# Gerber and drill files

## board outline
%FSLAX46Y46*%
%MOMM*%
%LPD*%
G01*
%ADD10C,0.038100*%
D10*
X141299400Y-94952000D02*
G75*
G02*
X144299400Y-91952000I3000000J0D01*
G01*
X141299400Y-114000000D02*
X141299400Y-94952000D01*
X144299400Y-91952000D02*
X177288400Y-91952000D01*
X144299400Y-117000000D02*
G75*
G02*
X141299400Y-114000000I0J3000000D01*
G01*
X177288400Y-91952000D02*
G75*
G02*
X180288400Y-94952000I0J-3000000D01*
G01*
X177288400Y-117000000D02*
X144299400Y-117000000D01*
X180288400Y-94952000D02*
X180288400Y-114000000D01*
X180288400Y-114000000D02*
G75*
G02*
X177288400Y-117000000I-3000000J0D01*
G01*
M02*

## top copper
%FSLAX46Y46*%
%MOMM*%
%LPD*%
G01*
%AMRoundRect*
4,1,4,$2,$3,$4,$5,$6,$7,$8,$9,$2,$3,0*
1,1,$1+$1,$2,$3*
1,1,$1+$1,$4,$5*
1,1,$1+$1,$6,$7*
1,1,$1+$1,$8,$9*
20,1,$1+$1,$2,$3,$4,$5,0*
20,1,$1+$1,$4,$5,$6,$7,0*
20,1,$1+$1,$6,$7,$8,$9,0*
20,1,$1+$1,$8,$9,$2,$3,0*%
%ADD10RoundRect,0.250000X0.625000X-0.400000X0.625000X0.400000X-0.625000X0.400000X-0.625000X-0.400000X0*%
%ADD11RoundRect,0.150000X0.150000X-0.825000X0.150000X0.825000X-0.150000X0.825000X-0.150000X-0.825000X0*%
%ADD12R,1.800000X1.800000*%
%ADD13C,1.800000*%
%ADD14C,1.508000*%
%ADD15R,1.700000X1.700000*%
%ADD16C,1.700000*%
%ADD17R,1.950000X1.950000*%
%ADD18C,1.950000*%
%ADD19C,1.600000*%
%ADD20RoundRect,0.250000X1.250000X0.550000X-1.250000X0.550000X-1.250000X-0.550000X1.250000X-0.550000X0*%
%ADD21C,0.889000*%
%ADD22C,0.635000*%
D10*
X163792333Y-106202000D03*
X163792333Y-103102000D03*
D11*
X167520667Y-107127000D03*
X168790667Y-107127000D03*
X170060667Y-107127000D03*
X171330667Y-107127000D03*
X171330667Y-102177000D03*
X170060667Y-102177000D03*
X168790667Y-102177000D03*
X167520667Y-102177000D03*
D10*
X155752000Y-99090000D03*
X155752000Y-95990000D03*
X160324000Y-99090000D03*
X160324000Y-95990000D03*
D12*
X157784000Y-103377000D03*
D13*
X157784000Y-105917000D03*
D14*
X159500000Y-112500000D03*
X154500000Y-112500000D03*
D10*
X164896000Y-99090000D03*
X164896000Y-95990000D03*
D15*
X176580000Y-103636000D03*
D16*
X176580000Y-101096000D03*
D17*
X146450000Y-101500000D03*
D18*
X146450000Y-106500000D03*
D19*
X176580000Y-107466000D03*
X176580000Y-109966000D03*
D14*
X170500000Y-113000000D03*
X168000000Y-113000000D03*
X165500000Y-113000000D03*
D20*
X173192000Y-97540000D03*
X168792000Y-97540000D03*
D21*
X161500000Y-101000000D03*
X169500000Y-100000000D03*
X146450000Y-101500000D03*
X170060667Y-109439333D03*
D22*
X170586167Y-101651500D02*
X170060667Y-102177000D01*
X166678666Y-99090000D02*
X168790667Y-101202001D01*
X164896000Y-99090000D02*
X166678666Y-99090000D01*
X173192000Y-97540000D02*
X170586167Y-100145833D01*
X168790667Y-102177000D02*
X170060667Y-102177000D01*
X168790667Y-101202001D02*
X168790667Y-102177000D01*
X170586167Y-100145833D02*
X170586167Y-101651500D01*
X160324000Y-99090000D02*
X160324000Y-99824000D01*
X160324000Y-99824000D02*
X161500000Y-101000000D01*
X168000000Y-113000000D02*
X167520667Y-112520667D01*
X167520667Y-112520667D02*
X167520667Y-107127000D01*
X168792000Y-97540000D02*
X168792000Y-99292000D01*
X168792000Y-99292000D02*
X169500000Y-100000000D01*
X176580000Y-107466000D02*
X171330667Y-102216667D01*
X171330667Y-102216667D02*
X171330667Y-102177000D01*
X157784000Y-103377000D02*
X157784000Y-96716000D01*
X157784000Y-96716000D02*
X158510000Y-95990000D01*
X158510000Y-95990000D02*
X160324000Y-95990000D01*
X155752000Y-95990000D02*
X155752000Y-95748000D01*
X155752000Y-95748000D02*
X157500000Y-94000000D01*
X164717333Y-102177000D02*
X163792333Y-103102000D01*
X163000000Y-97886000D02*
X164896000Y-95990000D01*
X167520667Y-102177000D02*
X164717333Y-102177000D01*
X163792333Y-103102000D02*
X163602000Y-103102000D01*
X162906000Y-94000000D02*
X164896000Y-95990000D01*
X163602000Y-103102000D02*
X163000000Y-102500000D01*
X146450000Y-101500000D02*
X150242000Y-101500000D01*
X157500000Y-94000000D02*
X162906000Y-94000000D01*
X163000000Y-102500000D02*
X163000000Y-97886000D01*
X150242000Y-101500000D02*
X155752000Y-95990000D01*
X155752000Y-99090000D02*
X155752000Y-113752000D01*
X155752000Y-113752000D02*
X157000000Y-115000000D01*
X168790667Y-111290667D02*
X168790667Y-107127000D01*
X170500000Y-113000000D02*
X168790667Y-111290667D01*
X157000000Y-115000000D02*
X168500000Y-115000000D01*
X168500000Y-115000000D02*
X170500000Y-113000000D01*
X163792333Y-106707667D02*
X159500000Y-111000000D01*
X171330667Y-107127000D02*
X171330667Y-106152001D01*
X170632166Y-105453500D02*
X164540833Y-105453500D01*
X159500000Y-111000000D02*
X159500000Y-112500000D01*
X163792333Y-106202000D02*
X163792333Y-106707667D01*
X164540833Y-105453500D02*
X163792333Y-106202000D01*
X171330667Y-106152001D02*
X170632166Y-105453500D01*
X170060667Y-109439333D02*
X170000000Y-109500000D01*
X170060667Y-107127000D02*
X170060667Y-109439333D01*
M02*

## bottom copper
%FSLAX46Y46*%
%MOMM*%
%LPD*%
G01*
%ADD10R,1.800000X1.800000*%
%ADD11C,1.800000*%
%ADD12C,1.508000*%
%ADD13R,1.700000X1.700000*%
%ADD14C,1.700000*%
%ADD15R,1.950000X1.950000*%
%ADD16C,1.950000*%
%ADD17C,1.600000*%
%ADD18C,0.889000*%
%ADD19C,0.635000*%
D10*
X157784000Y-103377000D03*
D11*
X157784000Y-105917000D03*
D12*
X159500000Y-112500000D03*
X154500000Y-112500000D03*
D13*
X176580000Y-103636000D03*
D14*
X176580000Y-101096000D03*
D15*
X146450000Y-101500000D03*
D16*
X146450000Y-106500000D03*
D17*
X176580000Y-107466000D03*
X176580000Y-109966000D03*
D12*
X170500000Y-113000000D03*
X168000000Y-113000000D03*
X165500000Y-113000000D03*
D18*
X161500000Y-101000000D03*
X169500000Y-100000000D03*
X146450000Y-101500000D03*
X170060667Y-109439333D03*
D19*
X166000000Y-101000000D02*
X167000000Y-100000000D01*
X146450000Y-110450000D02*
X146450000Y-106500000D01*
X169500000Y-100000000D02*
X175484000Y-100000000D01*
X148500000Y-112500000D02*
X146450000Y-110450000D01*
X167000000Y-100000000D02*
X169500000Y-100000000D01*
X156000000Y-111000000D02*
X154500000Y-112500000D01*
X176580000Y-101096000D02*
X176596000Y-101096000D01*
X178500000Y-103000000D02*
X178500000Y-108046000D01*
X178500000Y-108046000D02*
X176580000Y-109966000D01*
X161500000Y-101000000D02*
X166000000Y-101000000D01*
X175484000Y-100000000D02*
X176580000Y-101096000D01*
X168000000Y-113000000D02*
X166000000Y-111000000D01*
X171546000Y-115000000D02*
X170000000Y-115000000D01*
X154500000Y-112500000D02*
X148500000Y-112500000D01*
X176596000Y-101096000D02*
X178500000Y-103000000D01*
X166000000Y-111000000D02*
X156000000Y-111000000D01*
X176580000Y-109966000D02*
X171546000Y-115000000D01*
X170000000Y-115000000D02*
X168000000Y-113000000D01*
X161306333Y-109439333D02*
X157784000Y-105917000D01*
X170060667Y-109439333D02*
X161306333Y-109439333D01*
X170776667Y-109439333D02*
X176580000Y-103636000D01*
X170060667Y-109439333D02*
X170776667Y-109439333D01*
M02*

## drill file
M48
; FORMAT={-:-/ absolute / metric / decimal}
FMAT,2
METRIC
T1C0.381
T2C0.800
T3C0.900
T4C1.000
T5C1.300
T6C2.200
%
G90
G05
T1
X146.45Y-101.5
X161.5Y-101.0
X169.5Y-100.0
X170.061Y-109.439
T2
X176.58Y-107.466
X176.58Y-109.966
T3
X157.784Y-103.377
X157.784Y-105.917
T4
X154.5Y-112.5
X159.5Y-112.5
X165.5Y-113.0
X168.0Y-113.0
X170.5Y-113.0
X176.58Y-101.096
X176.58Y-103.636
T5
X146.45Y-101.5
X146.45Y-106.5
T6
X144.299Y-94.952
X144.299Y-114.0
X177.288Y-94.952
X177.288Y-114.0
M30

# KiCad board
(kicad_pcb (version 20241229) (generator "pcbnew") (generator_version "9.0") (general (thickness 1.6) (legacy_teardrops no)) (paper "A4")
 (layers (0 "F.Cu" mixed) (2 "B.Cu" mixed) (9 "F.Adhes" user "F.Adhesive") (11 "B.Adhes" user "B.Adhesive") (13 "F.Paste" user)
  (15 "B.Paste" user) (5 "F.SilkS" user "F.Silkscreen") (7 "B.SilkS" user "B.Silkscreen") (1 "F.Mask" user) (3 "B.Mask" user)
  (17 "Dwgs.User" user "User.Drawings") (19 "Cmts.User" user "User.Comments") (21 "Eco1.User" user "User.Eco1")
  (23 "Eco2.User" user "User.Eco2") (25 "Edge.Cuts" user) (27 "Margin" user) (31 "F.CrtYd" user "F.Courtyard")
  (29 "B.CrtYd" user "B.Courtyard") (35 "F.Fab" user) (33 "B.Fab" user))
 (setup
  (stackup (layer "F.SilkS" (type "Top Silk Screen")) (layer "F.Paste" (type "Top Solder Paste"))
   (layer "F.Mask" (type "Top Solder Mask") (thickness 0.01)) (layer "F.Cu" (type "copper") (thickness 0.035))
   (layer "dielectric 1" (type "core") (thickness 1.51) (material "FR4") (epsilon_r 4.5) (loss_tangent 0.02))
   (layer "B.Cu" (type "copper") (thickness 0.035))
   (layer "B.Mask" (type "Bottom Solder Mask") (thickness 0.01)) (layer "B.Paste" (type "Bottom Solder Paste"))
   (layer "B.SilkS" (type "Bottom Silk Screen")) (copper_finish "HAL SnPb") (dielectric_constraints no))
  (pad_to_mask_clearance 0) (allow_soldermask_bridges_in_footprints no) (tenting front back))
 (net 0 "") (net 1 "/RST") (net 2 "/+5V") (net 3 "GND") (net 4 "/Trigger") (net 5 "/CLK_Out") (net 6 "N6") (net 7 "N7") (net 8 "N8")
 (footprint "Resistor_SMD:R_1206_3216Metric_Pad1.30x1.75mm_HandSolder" (layer "F.Cu") (at 163.792333 104.652 90)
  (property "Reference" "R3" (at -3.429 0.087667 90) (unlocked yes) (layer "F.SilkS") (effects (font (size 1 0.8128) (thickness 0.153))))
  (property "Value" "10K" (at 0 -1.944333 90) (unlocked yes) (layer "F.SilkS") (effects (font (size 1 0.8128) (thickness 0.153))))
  (pad "1" smd roundrect (at -1.55 0 90) (size 1.3 1.75) (layers "F.Cu" "F.Mask" "F.Paste") (roundrect_rratio 0.192308) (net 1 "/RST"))
  (pad "2" smd roundrect (at 1.55 0 90) (size 1.3 1.75) (layers "F.Cu" "F.Mask" "F.Paste") (roundrect_rratio 0.192308) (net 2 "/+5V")))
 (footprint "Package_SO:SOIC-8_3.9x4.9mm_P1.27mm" (layer "F.Cu") (at 169.425667 104.652 90)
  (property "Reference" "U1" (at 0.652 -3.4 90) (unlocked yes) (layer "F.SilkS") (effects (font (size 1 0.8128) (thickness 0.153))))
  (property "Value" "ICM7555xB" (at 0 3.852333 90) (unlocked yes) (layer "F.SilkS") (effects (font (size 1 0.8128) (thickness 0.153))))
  (pad "1" smd roundrect (at -2.475 -1.905 90) (size 1.95 0.6) (layers "F.Cu" "F.Mask" "F.Paste") (roundrect_rratio 0.25) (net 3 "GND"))
  (pad "2" smd roundrect (at -2.475 -0.635 90) (size 1.95 0.6) (layers "F.Cu" "F.Mask" "F.Paste") (roundrect_rratio 0.25) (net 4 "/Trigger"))
  (pad "3" smd roundrect (at -2.475 0.635 90) (size 1.95 0.6) (layers "F.Cu" "F.Mask" "F.Paste") (roundrect_rratio 0.25) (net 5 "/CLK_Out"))
  (pad "4" smd roundrect (at -2.475 1.905 90) (size 1.95 0.6) (layers "F.Cu" "F.Mask" "F.Paste") (roundrect_rratio 0.25) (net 1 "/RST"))
  (pad "5" smd roundrect (at 2.475 1.905 90) (size 1.95 0.6) (layers "F.Cu" "F.Mask" "F.Paste") (roundrect_rratio 0.25) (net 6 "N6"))
  (pad "6" smd roundrect (at 2.475 0.635 90) (size 1.95 0.6) (layers "F.Cu" "F.Mask" "F.Paste") (roundrect_rratio 0.25) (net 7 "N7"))
  (pad "7" smd roundrect (at 2.475 -0.635 90) (size 1.95 0.6) (layers "F.Cu" "F.Mask" "F.Paste") (roundrect_rratio 0.25) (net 7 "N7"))
  (pad "8" smd roundrect (at 2.475 -1.905 90) (size 1.95 0.6) (layers "F.Cu" "F.Mask" "F.Paste") (roundrect_rratio 0.25) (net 2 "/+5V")))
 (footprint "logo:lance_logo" (layer "F.Cu") (at 149.5 95.5)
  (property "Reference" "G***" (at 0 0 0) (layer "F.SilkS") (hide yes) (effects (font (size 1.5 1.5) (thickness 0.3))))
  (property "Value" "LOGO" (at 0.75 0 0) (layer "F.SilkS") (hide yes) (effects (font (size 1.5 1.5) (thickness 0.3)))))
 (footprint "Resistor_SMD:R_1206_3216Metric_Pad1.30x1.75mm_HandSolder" (layer "F.Cu") (at 155.752 97.54 90)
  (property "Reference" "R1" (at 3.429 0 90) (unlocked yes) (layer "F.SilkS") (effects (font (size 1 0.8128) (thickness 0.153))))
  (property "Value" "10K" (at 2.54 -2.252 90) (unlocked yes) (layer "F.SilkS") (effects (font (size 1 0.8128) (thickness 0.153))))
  (pad "1" smd roundrect (at -1.55 0 90) (size 1.3 1.75) (layers "F.Cu" "F.Mask" "F.Paste") (roundrect_rratio 0.192308) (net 4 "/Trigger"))
  (pad "2" smd roundrect (at 1.55 0 90) (size 1.3 1.75) (layers "F.Cu" "F.Mask" "F.Paste") (roundrect_rratio 0.192308) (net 2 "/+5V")))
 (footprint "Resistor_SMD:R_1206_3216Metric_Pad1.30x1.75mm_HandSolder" (layer "F.Cu") (at 160.324 97.54 90)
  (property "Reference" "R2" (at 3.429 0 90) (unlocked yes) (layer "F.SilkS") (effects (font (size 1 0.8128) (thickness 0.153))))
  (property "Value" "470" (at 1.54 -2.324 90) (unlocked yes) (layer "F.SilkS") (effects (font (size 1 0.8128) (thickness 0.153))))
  (pad "1" smd roundrect (at -1.55 0 90) (size 1.3 1.75) (layers "F.Cu" "F.Mask" "F.Paste") (roundrect_rratio 0.192308) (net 3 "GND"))
  (pad "2" smd roundrect (at 1.55 0 90) (size 1.3 1.75) (layers "F.Cu" "F.Mask" "F.Paste") (roundrect_rratio 0.192308) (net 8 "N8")))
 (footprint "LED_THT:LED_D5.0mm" (layer "F.Cu") (at 157.784 103.377 -90)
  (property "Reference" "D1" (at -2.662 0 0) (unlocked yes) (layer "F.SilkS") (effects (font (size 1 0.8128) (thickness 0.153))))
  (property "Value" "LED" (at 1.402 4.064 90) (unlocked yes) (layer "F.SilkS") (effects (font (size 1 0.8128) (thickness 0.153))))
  (pad "1" thru_hole rect (at 0 0 270) (size 1.8 1.8) (drill 0.9) (layers "*.Cu" "*.Mask") (remove_unused_layers no) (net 8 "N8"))
  (pad "2" thru_hole circle (at 2.54 0 270) (size 1.8 1.8) (drill 0.9) (layers "*.Cu" "*.Mask") (remove_unused_layers no) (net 5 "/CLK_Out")))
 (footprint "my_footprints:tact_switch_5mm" (layer "F.Cu") (at 157 112.5 180)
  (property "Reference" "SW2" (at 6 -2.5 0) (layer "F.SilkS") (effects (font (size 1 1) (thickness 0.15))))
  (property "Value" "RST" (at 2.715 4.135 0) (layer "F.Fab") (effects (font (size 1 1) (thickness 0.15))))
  (pad "1" thru_hole circle (at -2.5 0 180) (size 1.508 1.508) (drill 1) (layers "*.Cu" "*.Mask") (remove_unused_layers no) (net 1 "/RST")
   (solder_mask_margin 0.102))
  (pad "2" thru_hole circle (at 2.5 0 180) (size 1.508 1.508) (drill 1) (layers "*.Cu" "*.Mask") (remove_unused_layers no) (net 3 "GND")
   (solder_mask_margin 0.102)))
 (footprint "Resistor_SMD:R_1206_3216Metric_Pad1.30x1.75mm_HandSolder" (layer "F.Cu") (at 164.896 97.54 90)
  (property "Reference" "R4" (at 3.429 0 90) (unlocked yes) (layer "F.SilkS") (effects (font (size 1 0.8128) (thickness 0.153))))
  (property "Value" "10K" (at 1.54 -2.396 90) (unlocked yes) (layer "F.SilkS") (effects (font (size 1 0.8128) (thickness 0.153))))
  (pad "1" smd roundrect (at -1.55 0 90) (size 1.3 1.75) (layers "F.Cu" "F.Mask" "F.Paste") (roundrect_rratio 0.192308) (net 7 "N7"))
  (pad "2" smd roundrect (at 1.55 0 90) (size 1.3 1.75) (layers "F.Cu" "F.Mask" "F.Paste") (roundrect_rratio 0.192308) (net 2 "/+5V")))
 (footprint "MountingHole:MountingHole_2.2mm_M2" (layer "F.Cu") (at 144.2994 94.952)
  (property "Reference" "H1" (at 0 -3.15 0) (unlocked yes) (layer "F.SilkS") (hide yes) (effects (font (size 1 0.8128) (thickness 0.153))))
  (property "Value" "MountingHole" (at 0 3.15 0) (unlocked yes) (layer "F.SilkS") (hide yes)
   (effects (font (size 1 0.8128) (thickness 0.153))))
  (pad "" np_thru_hole circle (at 0 0) (size 2.2 2.2) (drill 2.2) (layers "*.Cu" "*.Mask")))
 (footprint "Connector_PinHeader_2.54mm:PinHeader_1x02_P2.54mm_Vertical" (layer "F.Cu") (at 176.58 103.636 180)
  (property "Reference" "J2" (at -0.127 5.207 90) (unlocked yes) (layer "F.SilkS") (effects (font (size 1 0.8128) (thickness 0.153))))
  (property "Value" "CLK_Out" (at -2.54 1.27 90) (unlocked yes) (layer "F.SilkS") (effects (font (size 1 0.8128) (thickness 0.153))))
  (pad "1" thru_hole rect (at 0 0 180) (size 1.7 1.7) (drill 1) (layers "*.Cu" "*.Mask") (remove_unused_layers no) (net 5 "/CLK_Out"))
  (pad "2" thru_hole circle (at 0 2.54 180) (size 1.7 1.7) (drill 1) (layers "*.Cu" "*.Mask") (remove_unused_layers no) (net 3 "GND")))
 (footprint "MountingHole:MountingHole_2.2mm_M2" (layer "F.Cu") (at 177.2884 114)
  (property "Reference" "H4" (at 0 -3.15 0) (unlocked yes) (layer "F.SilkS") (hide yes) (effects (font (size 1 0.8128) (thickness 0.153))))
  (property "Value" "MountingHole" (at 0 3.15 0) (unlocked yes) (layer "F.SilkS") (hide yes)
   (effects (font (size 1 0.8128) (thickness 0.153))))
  (pad "" np_thru_hole circle (at 0 0) (size 2.2 2.2) (drill 2.2) (layers "*.Cu" "*.Mask")))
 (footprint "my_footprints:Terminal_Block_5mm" (layer "F.Cu") (at 146.45 104 -90)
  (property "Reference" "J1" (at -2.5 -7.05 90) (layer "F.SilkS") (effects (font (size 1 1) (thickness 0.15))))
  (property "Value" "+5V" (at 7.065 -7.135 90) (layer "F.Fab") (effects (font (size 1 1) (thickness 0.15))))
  (pad "1" thru_hole rect (at -2.5 0 270) (size 1.95 1.95) (drill 1.3) (layers "*.Cu" "*.Mask") (remove_unused_layers no) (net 2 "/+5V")
   (solder_mask_margin 0.102))
  (pad "2" thru_hole circle (at 2.5 0 270) (size 1.95 1.95) (drill 1.3) (layers "*.Cu" "*.Mask") (remove_unused_layers no) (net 3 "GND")
   (solder_mask_margin 0.102)))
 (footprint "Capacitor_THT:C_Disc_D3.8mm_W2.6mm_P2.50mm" (layer "F.Cu") (at 176.58 107.466 -90)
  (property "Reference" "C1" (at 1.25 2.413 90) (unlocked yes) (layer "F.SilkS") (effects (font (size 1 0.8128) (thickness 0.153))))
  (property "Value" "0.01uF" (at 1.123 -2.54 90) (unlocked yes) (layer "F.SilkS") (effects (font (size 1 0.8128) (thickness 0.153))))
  (pad "1" thru_hole circle (at 0 0 270) (size 1.6 1.6) (drill 0.8) (layers "*.Cu" "*.Mask") (remove_unused_layers no) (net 6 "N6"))
  (pad "2" thru_hole circle (at 2.5 0 270) (size 1.6 1.6) (drill 0.8) (layers "*.Cu" "*.Mask") (remove_unused_layers no) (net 3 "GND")))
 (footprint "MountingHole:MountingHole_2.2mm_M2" (layer "F.Cu") (at 177.2884 94.952)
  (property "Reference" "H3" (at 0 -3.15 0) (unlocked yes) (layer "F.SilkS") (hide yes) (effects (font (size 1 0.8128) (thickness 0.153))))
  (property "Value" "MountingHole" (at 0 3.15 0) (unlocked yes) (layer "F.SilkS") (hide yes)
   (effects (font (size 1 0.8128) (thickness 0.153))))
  (pad "" np_thru_hole circle (at 0 0) (size 2.2 2.2) (drill 2.2) (layers "*.Cu" "*.Mask")))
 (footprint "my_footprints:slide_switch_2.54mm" (layer "F.Cu") (at 168 113 180)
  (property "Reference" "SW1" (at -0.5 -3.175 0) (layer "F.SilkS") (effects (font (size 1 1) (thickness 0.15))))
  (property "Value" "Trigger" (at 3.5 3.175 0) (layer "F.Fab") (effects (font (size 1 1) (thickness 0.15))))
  (pad "1" thru_hole circle (at -2.5 0 180) (size 1.508 1.508) (drill 1) (layers "*.Cu" "*.Mask") (remove_unused_layers no)
   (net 4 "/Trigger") (solder_mask_margin 0.102))
  (pad "2" thru_hole circle (at 0 0 180) (size 1.508 1.508) (drill 1) (layers "*.Cu" "*.Mask") (remove_unused_layers no) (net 3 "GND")
   (solder_mask_margin 0.102))
  (pad "3" thru_hole circle (at 2.5 0 180) (size 1.508 1.508) (drill 1) (layers "*.Cu" "*.Mask") (remove_unused_layers no)
   (solder_mask_margin 0.102)))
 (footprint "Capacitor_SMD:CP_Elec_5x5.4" (layer "F.Cu") (at 170.992 97.54 180)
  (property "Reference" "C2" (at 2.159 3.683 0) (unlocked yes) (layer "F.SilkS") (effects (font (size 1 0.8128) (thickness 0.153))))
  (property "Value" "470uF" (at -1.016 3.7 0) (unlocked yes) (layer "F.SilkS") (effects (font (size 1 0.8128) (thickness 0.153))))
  (pad "1" smd roundrect (at -2.2 0 180) (size 3 1.6) (layers "F.Cu" "F.Mask" "F.Paste") (roundrect_rratio 0.15625) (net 7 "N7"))
  (pad "2" smd roundrect (at 2.2 0 180) (size 3 1.6) (layers "F.Cu" "F.Mask" "F.Paste") (roundrect_rratio 0.15625) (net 3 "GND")))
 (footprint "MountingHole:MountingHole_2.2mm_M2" (layer "F.Cu") (at 144.2994 114)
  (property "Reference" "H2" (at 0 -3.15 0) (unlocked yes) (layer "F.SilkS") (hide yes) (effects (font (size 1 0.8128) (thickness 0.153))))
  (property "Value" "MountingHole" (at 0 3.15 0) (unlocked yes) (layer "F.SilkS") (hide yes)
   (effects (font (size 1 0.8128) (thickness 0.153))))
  (pad "" np_thru_hole circle (at 0 0) (size 2.2 2.2) (drill 2.2) (layers "*.Cu" "*.Mask")))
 (gr_arc (start 141.2994 94.952) (mid 142.17808 92.83068) (end 144.2994 91.952) (stroke (width 0.0381) (type default)) (layer "Edge.Cuts"))
 (gr_line (start 141.2994 114) (end 141.2994 94.952) (stroke (width 0.0381) (type default)) (layer "Edge.Cuts"))
 (gr_line (start 144.2994 91.952) (end 177.2884 91.952) (stroke (width 0.0381) (type default)) (layer "Edge.Cuts"))
 (gr_arc (start 144.2994 117) (mid 142.17808 116.12132) (end 141.2994 114) (stroke (width 0.0381) (type default)) (layer "Edge.Cuts"))
 (gr_arc (start 177.2884 91.952) (mid 179.40972 92.83068) (end 180.2884 94.952) (stroke (width 0.0381) (type default)) (layer "Edge.Cuts"))
 (gr_line (start 177.2884 117) (end 144.2994 117) (stroke (width 0.0381) (type default)) (layer "Edge.Cuts"))
 (gr_line (start 180.2884 94.952) (end 180.2884 114) (stroke (width 0.0381) (type default)) (layer "Edge.Cuts"))
 (gr_arc (start 180.2884 114) (mid 179.40972 116.12132) (end 177.2884 117) (stroke (width 0.0381) (type default)) (layer "Edge.Cuts"))
 (segment (start 170.586167 101.6515) (end 170.060667 102.177) (width 0.635) (layer "F.Cu") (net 7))
 (segment (start 166.678666 99.09) (end 168.790667 101.202001) (width 0.635) (layer "F.Cu") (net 7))
 (segment (start 164.896 99.09) (end 166.678666 99.09) (width 0.635) (layer "F.Cu") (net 7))
 (segment (start 173.192 97.54) (end 170.586167 100.145833) (width 0.635) (layer "F.Cu") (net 7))
 (segment (start 168.790667 102.177) (end 170.060667 102.177) (width 0.635) (layer "F.Cu") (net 7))
 (segment (start 168.790667 101.202001) (end 168.790667 102.177) (width 0.635) (layer "F.Cu") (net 7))
 (segment (start 170.586167 100.145833) (end 170.586167 101.6515) (width 0.635) (layer "F.Cu") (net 7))
 (segment (start 160.324 99.09) (end 160.324 99.824) (width 0.635) (layer "F.Cu") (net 3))
 (segment (start 160.324 99.824) (end 161.5 101) (width 0.635) (layer "F.Cu") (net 3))
 (segment (start 168 113) (end 167.520667 112.520667) (width 0.635) (layer "F.Cu") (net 3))
 (segment (start 167.520667 112.520667) (end 167.520667 107.127) (width 0.635) (layer "F.Cu") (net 3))
 (segment (start 168.792 97.54) (end 168.792 99.292) (width 0.635) (layer "F.Cu") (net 3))
 (segment (start 168.792 99.292) (end 169.5 100) (width 0.635) (layer "F.Cu") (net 3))
 (via (at 161.5 101) (size 0.889) (drill 0.381) (layers "F.Cu" "B.Cu") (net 3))
 (via (at 169.5 100) (size 0.889) (drill 0.381) (layers "F.Cu" "B.Cu") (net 3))
 (segment (start 166 101) (end 167 100) (width 0.635) (layer "B.Cu") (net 3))
 (segment (start 146.45 110.45) (end 146.45 106.5) (width 0.635) (layer "B.Cu") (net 3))
 (segment (start 169.5 100) (end 175.484 100) (width 0.635) (layer "B.Cu") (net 3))
 (segment (start 148.5 112.5) (end 146.45 110.45) (width 0.635) (layer "B.Cu") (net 3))
 (segment (start 167 100) (end 169.5 100) (width 0.635) (layer "B.Cu") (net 3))
 (segment (start 156 111) (end 154.5 112.5) (width 0.635) (layer "B.Cu") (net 3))
 (segment (start 176.58 101.096) (end 176.596 101.096) (width 0.635) (layer "B.Cu") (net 3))
 (segment (start 178.5 103) (end 178.5 108.046) (width 0.635) (layer "B.Cu") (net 3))
 (segment (start 178.5 108.046) (end 176.58 109.966) (width 0.635) (layer "B.Cu") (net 3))
 (segment (start 161.5 101) (end 166 101) (width 0.635) (layer "B.Cu") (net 3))
 (segment (start 175.484 100) (end 176.58 101.096) (width 0.635) (layer "B.Cu") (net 3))
 (segment (start 168 113) (end 166 111) (width 0.635) (layer "B.Cu") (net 3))
 (segment (start 171.546 115) (end 170 115) (width 0.635) (layer "B.Cu") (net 3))
 (segment (start 154.5 112.5) (end 148.5 112.5) (width 0.635) (layer "B.Cu") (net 3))
 (segment (start 176.596 101.096) (end 178.5 103) (width 0.635) (layer "B.Cu") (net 3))
 (segment (start 166 111) (end 156 111) (width 0.635) (layer "B.Cu") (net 3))
 (segment (start 176.58 109.966) (end 171.546 115) (width 0.635) (layer "B.Cu") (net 3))
 (segment (start 170 115) (end 168 113) (width 0.635) (layer "B.Cu") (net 3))
 (segment (start 176.58 107.466) (end 171.330667 102.216667) (width 0.635) (layer "F.Cu") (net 6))
 (segment (start 171.330667 102.216667) (end 171.330667 102.177) (width 0.635) (layer "F.Cu") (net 6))
 (segment (start 157.784 103.377) (end 157.784 96.716) (width 0.635) (layer "F.Cu") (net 8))
 (segment (start 157.784 96.716) (end 158.51 95.99) (width 0.635) (layer "F.Cu") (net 8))
 (segment (start 158.51 95.99) (end 160.324 95.99) (width 0.635) (layer "F.Cu") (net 8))
 (segment (start 155.752 95.99) (end 155.752 95.748) (width 0.635) (layer "F.Cu") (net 2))
 (segment (start 155.752 95.748) (end 157.5 94) (width 0.635) (layer "F.Cu") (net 2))
 (segment (start 164.717333 102.177) (end 163.792333 103.102) (width 0.635) (layer "F.Cu") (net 2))
 (segment (start 163 97.886) (end 164.896 95.99) (width 0.635) (layer "F.Cu") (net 2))
 (segment (start 167.520667 102.177) (end 164.717333 102.177) (width 0.635) (layer "F.Cu") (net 2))
 (segment (start 163.792333 103.102) (end 163.602 103.102) (width 0.635) (layer "F.Cu") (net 2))
 (segment (start 162.906 94) (end 164.896 95.99) (width 0.635) (layer "F.Cu") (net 2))
 (segment (start 163.602 103.102) (end 163 102.5) (width 0.635) (layer "F.Cu") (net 2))
 (segment (start 146.45 101.5) (end 150.242 101.5) (width 0.635) (layer "F.Cu") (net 2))
 (segment (start 157.5 94) (end 162.906 94) (width 0.635) (layer "F.Cu") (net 2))
 (segment (start 163 102.5) (end 163 97.886) (width 0.635) (layer "F.Cu") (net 2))
 (segment (start 150.242 101.5) (end 155.752 95.99) (width 0.635) (layer "F.Cu") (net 2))
 (via (at 146.45 101.5) (size 0.889) (drill 0.381) (layers "F.Cu" "B.Cu") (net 2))
 (segment (start 155.752 99.09) (end 155.752 113.752) (width 0.635) (layer "F.Cu") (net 4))
 (segment (start 155.752 113.752) (end 157 115) (width 0.635) (layer "F.Cu") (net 4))
 (segment (start 168.790667 111.290667) (end 168.790667 107.127) (width 0.635) (layer "F.Cu") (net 4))
 (segment (start 170.5 113) (end 168.790667 111.290667) (width 0.635) (layer "F.Cu") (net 4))
 (segment (start 157 115) (end 168.5 115) (width 0.635) (layer "F.Cu") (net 4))
 (segment (start 168.5 115) (end 170.5 113) (width 0.635) (layer "F.Cu") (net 4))
 (segment (start 163.792333 106.707667) (end 159.5 111) (width 0.635) (layer "F.Cu") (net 1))
 (segment (start 171.330667 107.127) (end 171.330667 106.152001) (width 0.635) (layer "F.Cu") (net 1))
 (segment (start 170.632166 105.4535) (end 164.540833 105.4535) (width 0.635) (layer "F.Cu") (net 1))
 (segment (start 159.5 111) (end 159.5 112.5) (width 0.635) (layer "F.Cu") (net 1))
 (segment (start 163.792333 106.202) (end 163.792333 106.707667) (width 0.635) (layer "F.Cu") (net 1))
 (segment (start 164.540833 105.4535) (end 163.792333 106.202) (width 0.635) (layer "F.Cu") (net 1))
 (segment (start 171.330667 106.152001) (end 170.632166 105.4535) (width 0.635) (layer "F.Cu") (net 1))
 (segment (start 170.060667 109.439333) (end 170 109.5) (width 0.635) (layer "F.Cu") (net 5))
 (segment (start 170.060667 107.127) (end 170.060667 109.439333) (width 0.635) (layer "F.Cu") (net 5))
 (via (at 170.060667 109.439333) (size 0.889) (drill 0.381) (layers "F.Cu" "B.Cu") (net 5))
 (segment (start 161.306333 109.439333) (end 157.784 105.917) (width 0.635) (layer "B.Cu") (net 5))
 (segment (start 170.060667 109.439333) (end 161.306333 109.439333) (width 0.635) (layer "B.Cu") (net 5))
 (segment (start 170.776667 109.439333) (end 176.58 103.636) (width 0.635) (layer "B.Cu") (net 5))
 (segment (start 170.060667 109.439333) (end 170.776667 109.439333) (width 0.635) (layer "B.Cu") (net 5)))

